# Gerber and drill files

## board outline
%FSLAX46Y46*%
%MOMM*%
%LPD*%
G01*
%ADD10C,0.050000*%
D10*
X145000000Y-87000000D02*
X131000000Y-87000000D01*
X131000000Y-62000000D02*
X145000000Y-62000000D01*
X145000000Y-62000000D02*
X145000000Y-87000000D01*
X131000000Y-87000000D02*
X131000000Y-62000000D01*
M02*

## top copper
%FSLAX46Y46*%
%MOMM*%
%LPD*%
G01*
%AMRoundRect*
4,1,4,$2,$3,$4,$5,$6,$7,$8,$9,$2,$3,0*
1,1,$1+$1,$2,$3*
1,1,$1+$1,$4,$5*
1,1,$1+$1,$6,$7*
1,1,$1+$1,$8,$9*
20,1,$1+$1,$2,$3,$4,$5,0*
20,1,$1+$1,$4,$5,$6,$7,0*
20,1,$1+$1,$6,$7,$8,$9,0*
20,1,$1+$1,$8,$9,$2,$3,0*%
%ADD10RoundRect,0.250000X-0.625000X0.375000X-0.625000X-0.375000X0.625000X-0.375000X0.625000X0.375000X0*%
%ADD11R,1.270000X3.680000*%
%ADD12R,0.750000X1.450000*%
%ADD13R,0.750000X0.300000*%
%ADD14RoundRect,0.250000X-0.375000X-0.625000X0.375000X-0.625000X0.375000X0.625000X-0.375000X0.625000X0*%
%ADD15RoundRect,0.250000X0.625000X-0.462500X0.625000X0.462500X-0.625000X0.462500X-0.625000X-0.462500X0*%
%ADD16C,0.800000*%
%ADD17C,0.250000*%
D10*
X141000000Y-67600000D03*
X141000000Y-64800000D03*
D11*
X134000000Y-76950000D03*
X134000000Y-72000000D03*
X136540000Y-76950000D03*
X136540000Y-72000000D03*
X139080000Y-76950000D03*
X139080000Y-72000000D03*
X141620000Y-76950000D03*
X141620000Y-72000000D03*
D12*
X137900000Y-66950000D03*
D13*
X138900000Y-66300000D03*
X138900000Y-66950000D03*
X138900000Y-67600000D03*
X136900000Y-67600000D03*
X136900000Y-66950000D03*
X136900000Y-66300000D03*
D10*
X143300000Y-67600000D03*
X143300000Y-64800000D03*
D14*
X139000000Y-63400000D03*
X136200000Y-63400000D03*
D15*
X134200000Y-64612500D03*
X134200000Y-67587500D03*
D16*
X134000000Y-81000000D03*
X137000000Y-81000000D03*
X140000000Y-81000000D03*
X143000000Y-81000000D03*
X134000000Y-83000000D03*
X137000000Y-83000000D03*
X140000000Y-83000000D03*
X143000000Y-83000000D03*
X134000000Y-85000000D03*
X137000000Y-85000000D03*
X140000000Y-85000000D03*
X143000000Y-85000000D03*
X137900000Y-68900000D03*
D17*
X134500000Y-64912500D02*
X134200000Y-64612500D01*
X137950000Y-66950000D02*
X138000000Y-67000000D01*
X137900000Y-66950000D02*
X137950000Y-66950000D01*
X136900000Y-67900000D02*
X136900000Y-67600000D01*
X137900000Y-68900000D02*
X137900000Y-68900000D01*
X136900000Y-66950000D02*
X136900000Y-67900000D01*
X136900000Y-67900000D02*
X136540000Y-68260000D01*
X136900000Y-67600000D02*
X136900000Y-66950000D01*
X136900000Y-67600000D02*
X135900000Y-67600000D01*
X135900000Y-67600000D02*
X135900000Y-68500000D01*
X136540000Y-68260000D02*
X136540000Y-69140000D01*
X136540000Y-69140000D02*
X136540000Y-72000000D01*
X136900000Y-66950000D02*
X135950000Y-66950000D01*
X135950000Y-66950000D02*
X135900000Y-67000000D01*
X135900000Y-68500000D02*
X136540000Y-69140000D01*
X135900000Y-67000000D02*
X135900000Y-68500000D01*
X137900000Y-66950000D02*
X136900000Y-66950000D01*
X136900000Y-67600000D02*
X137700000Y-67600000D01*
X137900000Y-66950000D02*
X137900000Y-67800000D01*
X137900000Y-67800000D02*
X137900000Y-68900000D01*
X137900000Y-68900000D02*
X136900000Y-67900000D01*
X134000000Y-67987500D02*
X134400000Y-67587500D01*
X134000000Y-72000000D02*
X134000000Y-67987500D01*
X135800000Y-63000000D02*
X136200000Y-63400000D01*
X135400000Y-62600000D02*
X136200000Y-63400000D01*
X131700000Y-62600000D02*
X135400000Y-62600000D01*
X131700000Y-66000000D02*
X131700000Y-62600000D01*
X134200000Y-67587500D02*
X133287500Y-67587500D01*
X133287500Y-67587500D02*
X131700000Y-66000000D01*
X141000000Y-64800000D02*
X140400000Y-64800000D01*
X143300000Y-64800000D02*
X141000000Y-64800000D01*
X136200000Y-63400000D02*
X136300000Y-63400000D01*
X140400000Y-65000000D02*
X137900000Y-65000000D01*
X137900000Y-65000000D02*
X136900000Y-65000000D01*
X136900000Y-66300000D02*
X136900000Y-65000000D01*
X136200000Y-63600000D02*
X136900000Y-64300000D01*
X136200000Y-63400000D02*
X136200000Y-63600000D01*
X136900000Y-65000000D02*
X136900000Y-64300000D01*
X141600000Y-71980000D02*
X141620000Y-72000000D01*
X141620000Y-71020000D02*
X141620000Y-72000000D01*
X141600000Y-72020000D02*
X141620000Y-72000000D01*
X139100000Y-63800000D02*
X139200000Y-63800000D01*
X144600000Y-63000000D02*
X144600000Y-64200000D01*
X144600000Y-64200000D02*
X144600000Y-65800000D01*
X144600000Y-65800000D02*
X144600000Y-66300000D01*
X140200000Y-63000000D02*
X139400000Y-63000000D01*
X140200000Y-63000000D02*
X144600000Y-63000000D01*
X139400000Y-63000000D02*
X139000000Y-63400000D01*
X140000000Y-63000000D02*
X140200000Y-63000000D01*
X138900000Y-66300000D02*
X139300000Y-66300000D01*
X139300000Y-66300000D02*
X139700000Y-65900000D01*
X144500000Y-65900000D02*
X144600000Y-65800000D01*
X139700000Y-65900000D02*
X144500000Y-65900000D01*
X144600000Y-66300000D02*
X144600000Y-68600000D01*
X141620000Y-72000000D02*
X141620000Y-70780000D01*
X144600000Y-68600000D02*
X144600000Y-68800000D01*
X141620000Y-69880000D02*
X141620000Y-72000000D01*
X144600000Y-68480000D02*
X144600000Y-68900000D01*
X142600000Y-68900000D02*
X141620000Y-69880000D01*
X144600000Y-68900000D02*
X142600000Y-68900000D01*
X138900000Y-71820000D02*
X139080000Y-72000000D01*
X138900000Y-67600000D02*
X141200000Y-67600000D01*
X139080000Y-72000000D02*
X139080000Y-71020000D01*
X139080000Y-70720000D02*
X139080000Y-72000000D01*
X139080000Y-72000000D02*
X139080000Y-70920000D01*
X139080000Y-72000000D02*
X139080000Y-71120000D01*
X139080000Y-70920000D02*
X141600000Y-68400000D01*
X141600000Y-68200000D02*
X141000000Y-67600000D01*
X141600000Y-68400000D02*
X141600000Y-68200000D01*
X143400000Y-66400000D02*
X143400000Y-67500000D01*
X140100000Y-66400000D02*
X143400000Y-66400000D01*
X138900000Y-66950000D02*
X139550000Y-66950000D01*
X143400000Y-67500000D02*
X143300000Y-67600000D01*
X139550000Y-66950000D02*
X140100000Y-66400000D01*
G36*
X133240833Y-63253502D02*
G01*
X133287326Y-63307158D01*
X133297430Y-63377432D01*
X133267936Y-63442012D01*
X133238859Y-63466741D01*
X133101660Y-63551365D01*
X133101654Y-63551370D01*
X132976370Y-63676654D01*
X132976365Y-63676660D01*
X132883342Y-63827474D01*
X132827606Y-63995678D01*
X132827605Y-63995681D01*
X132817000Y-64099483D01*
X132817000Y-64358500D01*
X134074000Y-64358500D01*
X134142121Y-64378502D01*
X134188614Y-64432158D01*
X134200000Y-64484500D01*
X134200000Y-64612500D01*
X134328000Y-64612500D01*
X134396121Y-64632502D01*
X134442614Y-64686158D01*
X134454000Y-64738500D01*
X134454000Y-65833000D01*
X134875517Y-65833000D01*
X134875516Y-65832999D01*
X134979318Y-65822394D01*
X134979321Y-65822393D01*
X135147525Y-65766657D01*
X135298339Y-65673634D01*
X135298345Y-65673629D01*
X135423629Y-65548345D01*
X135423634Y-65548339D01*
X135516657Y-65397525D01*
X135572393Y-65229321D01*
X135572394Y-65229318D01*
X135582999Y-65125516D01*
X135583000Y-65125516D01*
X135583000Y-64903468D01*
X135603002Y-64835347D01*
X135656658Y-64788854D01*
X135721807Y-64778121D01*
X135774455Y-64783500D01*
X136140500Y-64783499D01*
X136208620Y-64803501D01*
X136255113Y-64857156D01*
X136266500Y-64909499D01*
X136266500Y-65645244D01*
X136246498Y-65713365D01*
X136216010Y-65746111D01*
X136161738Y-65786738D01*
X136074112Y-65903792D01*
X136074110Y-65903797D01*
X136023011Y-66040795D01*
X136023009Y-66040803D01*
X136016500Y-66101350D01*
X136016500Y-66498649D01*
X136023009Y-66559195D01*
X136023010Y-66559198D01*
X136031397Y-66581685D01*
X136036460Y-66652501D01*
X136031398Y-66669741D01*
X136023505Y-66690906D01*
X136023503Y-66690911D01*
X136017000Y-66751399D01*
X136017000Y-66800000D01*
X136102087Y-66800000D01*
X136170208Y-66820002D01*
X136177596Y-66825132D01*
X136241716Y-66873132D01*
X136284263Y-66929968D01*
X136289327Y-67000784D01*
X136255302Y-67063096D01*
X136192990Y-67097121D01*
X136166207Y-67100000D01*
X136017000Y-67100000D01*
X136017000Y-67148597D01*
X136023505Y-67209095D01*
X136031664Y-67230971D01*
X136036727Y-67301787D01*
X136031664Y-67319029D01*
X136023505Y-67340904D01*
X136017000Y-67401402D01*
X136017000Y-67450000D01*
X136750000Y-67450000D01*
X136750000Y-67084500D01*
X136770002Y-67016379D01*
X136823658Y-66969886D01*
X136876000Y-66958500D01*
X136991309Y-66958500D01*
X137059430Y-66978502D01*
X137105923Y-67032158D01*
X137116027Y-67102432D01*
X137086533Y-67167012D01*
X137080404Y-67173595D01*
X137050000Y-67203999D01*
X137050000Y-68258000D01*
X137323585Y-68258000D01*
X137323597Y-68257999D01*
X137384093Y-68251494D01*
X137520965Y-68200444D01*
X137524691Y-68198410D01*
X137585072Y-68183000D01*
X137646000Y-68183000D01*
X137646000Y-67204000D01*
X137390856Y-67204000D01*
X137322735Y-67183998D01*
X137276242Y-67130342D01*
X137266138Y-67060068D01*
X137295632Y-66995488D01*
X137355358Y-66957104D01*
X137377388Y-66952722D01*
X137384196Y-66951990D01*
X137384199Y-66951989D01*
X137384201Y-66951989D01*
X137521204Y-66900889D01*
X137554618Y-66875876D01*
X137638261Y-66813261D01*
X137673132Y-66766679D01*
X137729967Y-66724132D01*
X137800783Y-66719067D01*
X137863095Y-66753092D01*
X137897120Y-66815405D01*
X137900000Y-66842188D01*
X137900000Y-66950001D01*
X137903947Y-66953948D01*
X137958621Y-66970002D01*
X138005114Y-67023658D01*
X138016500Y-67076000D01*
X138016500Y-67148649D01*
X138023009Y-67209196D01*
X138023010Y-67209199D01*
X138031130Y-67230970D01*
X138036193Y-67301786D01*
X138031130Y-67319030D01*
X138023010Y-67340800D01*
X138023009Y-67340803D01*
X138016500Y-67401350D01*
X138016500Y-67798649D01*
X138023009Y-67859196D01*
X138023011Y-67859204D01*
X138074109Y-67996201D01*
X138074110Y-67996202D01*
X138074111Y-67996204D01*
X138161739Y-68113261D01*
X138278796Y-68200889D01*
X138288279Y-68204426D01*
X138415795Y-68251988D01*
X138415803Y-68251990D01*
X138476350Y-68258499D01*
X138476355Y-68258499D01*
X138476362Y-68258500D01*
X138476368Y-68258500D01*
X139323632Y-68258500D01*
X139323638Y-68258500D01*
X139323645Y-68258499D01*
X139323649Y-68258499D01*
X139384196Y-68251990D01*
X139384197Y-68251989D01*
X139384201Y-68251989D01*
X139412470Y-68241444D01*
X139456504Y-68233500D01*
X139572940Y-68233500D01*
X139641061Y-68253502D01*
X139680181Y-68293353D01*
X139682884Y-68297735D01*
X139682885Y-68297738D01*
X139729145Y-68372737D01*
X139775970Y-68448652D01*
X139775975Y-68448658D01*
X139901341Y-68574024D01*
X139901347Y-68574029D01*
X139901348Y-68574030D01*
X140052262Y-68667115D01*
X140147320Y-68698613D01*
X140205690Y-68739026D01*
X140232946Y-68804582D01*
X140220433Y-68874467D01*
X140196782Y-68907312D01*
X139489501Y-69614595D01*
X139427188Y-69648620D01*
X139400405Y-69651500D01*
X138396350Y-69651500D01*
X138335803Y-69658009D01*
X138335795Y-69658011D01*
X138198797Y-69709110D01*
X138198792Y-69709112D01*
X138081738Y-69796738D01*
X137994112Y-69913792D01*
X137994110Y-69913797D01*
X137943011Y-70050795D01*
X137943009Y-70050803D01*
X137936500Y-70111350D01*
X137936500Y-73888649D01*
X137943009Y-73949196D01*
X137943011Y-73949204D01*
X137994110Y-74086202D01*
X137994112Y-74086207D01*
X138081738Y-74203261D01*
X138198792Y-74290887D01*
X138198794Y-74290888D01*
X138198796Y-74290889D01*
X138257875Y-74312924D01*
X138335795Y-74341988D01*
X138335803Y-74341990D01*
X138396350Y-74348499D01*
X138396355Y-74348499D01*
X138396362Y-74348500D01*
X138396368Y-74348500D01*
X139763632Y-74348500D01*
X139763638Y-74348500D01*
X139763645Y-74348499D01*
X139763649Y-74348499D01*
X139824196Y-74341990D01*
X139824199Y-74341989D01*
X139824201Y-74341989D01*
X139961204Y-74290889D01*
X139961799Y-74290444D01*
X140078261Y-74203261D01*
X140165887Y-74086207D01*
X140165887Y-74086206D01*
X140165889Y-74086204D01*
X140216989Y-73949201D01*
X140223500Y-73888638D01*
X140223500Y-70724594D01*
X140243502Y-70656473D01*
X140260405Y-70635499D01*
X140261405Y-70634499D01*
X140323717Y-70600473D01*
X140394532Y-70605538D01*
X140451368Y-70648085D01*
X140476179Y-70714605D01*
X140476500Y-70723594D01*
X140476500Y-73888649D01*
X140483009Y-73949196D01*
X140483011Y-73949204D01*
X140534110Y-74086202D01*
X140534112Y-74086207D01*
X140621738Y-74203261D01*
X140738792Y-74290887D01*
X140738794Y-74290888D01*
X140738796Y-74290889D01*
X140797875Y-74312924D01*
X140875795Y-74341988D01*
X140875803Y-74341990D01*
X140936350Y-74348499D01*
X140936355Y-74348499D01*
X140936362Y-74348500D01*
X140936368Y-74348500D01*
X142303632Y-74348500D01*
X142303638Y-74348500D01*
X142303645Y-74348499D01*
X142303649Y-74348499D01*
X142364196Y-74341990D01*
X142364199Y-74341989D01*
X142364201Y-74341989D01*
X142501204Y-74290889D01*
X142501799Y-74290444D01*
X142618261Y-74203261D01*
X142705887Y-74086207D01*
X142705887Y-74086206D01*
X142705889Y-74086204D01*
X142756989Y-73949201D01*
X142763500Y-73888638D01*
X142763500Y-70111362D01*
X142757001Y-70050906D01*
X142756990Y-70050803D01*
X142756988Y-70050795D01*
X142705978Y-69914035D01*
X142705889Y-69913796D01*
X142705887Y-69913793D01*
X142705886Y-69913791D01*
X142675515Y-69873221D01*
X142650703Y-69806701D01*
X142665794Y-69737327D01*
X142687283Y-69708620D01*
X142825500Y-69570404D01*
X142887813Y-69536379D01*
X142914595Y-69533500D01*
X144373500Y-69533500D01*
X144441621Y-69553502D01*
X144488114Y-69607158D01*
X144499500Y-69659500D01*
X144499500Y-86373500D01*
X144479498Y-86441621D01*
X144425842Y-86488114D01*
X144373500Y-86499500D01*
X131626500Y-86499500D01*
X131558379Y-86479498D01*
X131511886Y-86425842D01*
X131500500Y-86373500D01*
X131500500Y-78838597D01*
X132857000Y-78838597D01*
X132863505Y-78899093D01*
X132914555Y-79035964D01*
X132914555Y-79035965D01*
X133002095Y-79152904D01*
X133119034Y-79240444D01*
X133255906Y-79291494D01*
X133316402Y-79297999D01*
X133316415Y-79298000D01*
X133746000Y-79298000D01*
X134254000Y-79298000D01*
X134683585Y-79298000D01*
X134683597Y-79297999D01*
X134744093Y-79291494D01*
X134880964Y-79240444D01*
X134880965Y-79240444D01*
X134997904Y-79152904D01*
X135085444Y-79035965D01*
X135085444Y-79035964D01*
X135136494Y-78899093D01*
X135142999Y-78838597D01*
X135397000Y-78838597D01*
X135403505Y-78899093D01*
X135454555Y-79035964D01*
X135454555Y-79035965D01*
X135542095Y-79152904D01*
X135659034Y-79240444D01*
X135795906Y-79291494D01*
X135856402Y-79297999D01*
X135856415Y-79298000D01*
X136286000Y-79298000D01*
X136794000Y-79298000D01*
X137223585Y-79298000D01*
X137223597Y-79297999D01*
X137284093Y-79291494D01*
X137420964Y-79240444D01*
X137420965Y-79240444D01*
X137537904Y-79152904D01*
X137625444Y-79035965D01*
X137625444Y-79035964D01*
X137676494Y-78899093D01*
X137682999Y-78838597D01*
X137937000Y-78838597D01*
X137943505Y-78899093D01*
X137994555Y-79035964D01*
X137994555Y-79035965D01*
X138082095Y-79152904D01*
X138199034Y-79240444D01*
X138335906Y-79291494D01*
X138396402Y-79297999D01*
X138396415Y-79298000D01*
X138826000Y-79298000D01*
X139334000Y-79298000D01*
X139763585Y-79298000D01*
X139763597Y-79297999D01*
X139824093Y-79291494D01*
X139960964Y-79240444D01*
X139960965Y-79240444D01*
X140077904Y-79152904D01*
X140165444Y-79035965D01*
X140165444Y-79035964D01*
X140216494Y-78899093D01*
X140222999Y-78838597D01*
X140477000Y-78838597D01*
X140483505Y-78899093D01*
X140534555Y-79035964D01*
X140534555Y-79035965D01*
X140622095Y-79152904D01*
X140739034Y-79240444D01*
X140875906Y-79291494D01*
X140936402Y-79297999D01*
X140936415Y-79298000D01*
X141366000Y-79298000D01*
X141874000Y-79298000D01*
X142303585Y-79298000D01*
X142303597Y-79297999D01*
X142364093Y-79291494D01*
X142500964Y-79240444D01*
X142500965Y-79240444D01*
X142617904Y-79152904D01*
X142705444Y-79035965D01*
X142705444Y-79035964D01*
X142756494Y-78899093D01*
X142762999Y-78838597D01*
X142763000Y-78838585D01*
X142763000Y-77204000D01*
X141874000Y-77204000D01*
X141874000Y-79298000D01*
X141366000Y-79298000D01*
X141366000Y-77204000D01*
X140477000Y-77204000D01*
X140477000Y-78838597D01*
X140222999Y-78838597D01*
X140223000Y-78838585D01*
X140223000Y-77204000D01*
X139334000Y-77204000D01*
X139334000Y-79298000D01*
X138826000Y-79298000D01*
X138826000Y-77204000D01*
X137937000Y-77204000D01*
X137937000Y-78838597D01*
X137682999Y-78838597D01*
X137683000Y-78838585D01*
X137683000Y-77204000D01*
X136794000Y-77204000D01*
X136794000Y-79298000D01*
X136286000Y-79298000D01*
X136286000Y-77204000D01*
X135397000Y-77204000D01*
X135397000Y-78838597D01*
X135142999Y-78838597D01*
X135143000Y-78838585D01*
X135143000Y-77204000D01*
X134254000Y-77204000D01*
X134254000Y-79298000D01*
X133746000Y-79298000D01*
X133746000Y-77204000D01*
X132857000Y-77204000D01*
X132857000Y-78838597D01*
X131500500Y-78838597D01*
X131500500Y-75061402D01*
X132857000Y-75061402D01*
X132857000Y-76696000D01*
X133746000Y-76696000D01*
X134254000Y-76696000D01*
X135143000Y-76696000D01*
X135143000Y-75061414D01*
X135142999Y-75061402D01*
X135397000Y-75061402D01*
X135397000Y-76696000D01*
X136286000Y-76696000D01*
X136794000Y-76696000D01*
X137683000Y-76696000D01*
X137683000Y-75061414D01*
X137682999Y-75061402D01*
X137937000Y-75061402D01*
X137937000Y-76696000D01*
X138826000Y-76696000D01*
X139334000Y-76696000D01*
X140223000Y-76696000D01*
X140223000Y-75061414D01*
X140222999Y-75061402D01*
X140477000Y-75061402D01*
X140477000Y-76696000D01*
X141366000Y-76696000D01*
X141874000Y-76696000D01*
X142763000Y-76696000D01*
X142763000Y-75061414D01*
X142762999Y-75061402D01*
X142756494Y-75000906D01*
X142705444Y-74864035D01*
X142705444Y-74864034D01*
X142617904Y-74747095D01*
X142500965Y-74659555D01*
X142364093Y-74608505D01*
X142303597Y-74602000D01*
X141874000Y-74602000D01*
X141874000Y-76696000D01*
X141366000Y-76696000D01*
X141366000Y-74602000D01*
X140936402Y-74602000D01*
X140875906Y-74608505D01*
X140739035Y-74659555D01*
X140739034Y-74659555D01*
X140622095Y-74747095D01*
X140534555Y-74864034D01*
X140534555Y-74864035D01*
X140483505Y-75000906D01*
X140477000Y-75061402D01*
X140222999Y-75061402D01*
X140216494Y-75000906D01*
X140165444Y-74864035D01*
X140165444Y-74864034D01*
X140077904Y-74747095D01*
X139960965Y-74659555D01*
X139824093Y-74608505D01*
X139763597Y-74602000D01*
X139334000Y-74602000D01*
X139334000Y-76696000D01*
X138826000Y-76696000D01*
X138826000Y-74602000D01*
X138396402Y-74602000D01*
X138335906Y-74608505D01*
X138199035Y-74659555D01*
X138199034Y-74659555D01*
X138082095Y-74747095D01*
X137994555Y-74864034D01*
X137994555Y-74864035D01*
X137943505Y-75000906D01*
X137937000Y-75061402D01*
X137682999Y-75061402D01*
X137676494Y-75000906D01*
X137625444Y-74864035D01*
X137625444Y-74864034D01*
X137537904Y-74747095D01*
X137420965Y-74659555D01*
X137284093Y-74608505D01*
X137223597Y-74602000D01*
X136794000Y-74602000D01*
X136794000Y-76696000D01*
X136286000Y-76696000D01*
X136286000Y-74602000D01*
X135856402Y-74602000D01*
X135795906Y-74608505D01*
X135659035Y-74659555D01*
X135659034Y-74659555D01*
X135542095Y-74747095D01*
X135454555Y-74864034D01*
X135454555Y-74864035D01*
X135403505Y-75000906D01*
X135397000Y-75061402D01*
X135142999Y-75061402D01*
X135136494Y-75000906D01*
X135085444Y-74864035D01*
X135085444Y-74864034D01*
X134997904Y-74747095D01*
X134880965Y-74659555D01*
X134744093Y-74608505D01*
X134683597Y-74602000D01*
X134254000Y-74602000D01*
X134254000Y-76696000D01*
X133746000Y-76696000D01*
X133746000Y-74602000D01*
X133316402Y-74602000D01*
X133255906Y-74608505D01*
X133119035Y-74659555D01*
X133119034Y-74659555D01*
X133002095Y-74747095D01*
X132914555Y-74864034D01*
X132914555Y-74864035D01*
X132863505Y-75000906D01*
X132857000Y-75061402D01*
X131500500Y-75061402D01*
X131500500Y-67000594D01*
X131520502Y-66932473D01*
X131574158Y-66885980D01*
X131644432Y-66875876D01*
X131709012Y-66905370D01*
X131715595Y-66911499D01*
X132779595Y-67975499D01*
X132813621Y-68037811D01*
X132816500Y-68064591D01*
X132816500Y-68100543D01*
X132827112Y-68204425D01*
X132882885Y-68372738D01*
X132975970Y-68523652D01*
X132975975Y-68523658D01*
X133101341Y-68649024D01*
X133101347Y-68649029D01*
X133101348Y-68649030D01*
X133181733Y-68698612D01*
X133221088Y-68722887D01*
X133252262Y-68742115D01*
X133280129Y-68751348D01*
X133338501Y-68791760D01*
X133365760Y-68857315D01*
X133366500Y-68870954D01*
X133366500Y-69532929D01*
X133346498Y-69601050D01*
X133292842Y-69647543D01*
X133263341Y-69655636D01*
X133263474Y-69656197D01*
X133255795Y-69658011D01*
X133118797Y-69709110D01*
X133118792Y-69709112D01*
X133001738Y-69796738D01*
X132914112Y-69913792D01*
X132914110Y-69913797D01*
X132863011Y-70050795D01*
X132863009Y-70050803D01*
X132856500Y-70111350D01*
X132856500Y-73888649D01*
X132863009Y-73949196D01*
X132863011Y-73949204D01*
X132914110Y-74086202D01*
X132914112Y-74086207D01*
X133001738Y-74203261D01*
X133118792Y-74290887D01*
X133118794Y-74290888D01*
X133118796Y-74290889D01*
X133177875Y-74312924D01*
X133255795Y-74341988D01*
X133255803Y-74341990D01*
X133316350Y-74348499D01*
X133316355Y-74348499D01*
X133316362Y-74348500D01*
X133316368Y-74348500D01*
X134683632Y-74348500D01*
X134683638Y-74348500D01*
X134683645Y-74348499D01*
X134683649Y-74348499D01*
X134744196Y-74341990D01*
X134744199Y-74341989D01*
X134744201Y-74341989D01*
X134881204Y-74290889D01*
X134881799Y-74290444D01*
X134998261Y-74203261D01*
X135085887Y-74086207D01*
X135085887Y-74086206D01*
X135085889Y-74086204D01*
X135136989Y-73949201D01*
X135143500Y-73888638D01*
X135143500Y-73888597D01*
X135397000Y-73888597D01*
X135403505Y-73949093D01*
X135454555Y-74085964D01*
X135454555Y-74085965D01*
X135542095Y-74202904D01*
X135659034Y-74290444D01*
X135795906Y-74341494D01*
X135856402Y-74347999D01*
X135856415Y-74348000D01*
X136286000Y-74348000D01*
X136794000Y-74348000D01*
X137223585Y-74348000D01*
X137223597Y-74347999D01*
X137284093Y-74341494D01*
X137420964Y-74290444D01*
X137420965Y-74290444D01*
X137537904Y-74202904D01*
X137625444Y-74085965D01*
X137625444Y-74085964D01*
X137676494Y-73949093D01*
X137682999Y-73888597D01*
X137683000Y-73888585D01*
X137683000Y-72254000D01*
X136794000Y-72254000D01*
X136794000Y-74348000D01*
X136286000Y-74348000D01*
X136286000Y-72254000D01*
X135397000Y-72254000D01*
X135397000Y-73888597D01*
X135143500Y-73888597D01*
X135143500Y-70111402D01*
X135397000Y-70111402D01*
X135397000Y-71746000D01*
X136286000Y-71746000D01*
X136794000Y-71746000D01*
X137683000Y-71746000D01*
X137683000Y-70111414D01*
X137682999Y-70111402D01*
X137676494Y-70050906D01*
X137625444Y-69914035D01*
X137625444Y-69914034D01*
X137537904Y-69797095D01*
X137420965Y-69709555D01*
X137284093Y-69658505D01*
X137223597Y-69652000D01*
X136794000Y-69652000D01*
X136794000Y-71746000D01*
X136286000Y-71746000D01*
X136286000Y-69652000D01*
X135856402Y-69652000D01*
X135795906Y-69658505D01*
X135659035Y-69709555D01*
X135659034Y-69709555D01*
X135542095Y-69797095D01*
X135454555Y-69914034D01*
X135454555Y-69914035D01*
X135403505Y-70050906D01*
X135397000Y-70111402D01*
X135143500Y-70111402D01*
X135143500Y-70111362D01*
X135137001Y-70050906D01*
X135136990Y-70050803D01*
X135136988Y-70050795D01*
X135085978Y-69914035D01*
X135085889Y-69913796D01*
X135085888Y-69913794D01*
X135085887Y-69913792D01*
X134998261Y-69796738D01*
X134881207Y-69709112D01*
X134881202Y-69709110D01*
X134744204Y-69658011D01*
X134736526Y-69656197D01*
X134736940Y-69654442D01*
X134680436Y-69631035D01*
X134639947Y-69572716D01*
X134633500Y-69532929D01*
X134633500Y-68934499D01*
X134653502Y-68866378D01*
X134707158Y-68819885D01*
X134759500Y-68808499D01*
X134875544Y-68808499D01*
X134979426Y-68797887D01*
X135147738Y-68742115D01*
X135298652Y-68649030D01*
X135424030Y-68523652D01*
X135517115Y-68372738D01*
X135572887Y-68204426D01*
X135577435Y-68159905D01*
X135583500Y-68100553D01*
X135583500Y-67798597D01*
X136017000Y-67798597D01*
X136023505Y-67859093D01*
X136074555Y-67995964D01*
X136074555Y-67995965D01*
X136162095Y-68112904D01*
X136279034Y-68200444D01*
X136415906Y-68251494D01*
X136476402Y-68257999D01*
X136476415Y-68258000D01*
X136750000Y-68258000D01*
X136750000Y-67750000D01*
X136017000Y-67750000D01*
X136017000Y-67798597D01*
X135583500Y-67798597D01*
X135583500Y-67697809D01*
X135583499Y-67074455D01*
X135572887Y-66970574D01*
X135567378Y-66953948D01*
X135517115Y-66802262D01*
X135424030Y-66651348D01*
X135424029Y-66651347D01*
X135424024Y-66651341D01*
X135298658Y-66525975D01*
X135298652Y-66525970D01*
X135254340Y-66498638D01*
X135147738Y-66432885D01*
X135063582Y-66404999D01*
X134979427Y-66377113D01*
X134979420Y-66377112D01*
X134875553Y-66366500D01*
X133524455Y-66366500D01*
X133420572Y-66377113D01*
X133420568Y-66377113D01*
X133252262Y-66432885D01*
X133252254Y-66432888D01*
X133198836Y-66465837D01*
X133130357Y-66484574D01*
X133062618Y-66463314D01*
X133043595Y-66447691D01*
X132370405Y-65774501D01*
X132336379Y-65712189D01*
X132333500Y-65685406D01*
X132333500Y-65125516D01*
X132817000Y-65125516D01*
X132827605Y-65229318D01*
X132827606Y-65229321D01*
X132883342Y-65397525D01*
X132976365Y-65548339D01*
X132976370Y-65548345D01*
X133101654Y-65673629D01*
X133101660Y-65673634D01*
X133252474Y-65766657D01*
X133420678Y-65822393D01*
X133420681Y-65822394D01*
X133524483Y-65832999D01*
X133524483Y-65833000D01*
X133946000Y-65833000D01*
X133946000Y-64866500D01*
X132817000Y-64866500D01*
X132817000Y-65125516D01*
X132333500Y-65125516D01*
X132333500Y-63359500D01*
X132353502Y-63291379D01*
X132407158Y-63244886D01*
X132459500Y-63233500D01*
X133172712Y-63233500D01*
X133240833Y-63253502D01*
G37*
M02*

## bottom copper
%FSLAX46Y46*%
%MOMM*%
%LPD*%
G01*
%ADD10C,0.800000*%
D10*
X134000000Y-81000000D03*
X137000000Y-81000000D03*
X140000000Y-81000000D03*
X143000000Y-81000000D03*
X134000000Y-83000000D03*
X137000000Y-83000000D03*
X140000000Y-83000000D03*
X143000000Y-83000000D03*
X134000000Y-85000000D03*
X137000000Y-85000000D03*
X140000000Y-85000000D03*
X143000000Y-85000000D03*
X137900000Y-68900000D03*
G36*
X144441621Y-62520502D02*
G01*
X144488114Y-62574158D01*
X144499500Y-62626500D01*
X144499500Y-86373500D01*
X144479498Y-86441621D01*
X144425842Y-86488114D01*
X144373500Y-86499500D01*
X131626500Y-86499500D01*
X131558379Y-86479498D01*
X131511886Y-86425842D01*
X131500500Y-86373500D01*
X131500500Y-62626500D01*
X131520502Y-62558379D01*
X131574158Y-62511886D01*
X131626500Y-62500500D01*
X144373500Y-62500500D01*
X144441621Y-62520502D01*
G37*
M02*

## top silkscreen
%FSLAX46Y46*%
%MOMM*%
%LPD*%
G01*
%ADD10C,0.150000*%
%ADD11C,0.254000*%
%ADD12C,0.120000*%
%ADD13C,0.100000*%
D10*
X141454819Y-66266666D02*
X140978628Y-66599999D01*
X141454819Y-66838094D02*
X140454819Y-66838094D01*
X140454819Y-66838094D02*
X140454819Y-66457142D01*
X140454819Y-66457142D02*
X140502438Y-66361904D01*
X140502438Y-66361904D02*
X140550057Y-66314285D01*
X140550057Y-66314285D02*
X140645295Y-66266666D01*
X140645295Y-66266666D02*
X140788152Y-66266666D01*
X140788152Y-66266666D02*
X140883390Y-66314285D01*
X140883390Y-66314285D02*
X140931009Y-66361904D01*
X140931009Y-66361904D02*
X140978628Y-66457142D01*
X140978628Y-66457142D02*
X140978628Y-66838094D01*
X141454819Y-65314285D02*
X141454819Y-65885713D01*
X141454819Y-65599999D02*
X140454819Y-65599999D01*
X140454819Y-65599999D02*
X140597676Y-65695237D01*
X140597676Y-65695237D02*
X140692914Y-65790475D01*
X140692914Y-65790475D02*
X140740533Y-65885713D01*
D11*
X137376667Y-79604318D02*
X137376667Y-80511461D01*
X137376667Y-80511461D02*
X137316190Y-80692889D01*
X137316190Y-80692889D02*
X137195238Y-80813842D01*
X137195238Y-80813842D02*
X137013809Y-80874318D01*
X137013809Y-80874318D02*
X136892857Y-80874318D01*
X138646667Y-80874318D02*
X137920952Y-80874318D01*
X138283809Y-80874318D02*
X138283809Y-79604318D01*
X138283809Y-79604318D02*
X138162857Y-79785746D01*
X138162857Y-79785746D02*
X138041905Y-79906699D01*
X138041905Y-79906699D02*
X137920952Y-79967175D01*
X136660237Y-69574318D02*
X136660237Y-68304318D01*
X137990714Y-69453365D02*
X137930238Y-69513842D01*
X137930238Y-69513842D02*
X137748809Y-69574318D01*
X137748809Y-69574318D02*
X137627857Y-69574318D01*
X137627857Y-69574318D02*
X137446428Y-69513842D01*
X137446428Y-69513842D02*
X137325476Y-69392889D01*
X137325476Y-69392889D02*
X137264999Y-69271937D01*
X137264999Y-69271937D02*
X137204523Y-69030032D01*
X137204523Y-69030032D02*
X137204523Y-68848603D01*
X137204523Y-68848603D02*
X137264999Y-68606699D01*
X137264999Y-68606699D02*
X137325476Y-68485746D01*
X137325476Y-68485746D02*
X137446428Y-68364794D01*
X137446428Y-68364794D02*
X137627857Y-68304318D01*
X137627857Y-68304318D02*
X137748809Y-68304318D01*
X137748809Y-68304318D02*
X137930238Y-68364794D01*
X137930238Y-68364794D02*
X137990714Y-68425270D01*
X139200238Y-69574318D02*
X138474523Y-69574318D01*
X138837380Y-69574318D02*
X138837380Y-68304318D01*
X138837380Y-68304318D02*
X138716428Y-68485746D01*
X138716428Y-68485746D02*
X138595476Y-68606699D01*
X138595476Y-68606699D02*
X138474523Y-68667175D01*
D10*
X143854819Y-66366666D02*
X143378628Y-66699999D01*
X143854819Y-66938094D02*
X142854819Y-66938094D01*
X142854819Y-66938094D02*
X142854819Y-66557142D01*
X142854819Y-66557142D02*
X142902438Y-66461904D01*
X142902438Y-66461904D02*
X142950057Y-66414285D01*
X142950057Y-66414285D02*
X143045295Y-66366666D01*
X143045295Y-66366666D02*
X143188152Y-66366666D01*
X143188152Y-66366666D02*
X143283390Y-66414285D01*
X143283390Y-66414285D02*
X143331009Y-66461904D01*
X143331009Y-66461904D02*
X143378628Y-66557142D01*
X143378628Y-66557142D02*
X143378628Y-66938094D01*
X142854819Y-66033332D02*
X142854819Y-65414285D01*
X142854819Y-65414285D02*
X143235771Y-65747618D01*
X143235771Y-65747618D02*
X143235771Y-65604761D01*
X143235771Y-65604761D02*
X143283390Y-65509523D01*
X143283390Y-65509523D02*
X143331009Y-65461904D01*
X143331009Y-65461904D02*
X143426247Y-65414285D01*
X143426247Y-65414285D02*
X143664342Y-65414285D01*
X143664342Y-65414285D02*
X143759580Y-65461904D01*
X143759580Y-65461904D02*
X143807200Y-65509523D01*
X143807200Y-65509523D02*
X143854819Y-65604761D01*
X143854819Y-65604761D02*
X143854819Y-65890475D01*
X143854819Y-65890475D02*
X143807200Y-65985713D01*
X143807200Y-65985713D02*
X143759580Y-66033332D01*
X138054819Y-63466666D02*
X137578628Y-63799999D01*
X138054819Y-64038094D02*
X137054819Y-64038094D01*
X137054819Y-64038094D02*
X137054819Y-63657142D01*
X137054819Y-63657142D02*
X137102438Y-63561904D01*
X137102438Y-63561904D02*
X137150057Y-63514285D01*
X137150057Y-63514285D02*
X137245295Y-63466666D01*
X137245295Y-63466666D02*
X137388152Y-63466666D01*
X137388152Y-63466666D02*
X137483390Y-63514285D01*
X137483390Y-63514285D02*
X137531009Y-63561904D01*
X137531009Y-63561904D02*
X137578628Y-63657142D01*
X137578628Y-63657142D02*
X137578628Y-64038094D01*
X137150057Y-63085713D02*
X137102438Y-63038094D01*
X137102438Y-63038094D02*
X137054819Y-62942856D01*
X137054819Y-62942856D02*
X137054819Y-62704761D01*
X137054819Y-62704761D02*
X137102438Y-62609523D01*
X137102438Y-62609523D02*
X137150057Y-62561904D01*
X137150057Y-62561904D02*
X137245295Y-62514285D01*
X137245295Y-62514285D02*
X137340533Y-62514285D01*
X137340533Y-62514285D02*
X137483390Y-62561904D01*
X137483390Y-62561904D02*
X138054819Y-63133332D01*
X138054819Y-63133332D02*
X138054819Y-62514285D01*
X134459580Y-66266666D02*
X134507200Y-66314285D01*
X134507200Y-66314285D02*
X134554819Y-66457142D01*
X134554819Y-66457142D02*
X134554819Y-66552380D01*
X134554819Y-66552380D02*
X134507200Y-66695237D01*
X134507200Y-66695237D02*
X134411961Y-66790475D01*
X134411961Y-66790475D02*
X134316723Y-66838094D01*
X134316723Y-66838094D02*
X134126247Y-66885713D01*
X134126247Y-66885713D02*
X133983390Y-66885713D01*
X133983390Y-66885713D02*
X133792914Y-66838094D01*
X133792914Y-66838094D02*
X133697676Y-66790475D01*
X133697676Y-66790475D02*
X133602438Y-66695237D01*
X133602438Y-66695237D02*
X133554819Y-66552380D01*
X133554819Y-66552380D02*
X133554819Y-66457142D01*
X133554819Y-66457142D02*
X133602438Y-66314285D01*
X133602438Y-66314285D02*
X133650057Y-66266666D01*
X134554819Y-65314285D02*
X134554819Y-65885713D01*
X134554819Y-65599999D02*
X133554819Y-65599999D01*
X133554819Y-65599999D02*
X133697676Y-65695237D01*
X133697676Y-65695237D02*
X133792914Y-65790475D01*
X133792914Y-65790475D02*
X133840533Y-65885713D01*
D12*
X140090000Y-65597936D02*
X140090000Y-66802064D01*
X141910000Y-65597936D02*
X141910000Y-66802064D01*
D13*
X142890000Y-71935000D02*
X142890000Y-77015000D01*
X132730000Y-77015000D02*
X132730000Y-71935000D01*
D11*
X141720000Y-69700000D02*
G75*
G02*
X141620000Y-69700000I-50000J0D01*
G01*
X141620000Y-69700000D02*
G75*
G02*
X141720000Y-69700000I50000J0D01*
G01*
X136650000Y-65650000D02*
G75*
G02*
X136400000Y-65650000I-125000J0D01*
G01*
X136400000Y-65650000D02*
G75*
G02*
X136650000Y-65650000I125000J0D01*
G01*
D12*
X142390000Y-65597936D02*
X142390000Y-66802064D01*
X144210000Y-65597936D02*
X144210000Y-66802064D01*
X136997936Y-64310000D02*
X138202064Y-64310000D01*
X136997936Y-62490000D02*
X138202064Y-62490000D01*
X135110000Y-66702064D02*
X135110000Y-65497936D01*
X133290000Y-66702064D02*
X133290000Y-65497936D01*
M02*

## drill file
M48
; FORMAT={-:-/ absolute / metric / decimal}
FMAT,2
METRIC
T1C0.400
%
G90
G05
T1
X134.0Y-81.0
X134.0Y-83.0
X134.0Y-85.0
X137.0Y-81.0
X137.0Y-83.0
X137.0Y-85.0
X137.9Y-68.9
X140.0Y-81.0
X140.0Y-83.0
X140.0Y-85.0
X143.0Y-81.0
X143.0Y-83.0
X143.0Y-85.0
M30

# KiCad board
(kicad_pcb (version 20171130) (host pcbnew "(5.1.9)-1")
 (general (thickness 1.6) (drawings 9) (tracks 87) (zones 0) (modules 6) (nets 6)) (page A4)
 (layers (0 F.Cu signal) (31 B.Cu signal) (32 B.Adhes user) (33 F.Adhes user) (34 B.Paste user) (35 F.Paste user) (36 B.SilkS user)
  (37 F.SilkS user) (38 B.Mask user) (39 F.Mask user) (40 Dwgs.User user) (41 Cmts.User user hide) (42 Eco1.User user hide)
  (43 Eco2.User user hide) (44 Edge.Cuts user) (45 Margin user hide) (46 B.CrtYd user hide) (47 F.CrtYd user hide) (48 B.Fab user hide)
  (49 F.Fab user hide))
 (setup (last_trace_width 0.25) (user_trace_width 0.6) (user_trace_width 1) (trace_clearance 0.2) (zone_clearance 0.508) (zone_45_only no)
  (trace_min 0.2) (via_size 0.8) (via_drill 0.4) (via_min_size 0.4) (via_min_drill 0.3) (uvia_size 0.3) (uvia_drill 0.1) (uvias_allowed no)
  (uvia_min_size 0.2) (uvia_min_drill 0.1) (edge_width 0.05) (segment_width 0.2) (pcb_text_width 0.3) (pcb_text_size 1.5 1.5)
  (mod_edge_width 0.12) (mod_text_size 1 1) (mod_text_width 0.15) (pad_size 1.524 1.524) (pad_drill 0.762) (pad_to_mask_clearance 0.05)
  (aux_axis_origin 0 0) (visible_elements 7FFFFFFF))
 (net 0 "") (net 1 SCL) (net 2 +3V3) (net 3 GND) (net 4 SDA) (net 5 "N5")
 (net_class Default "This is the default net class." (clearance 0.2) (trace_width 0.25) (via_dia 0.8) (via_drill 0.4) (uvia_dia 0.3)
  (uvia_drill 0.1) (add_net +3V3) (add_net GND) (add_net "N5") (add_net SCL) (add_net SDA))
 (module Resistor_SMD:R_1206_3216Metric (layer F.Cu) (at 141 66.2 270)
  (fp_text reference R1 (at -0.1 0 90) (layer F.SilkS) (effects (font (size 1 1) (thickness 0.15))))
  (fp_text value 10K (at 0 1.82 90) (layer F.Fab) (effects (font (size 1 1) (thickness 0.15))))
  (fp_line (start -0.602064 0.91) (end 0.602064 0.91) (layer F.SilkS) (width 0.12))
  (fp_line (start -0.602064 -0.91) (end 0.602064 -0.91) (layer F.SilkS) (width 0.12))
  (pad 2 smd roundrect (at 1.4 0 270) (size 1.25 1.75) (layers F.Cu F.Paste F.Mask) (roundrect_rratio 0.2) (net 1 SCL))
  (pad 1 smd roundrect (at -1.4 0 270) (size 1.25 1.75) (layers F.Cu F.Paste F.Mask) (roundrect_rratio 0.2) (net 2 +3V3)))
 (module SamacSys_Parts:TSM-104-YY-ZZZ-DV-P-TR (layer F.Cu) (at 137.81 74.475)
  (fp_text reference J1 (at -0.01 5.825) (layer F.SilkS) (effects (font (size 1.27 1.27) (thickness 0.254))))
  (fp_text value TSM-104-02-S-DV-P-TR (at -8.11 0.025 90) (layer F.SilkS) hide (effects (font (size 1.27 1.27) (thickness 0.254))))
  (fp_line (start 5.08 -2.54) (end 5.08 2.54) (layer F.SilkS) (width 0.1))
  (fp_line (start -5.08 2.54) (end -5.08 -2.54) (layer F.SilkS) (width 0.1))
  (fp_circle (center 3.86 -4.775) (end 3.81 -4.775) (layer F.SilkS) (width 0.254))
  (pad 8 smd rect (at -3.81 2.475) (size 1.27 3.68) (layers F.Cu F.Paste F.Mask) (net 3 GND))
  (pad 7 smd rect (at -3.81 -2.475) (size 1.27 3.68) (layers F.Cu F.Paste F.Mask) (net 2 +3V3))
  (pad 6 smd rect (at -1.27 2.475) (size 1.27 3.68) (layers F.Cu F.Paste F.Mask) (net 3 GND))
  (pad 5 smd rect (at -1.27 -2.475) (size 1.27 3.68) (layers F.Cu F.Paste F.Mask) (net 3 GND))
  (pad 4 smd rect (at 1.27 2.475) (size 1.27 3.68) (layers F.Cu F.Paste F.Mask) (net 3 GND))
  (pad 3 smd rect (at 1.27 -2.475) (size 1.27 3.68) (layers F.Cu F.Paste F.Mask) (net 1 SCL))
  (pad 2 smd rect (at 3.81 2.475) (size 1.27 3.68) (layers F.Cu F.Paste F.Mask) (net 3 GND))
  (pad 1 smd rect (at 3.81 -2.475) (size 1.27 3.68) (layers F.Cu F.Paste F.Mask) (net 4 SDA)))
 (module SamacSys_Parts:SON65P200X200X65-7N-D (layer F.Cu) (at 137.9 66.95)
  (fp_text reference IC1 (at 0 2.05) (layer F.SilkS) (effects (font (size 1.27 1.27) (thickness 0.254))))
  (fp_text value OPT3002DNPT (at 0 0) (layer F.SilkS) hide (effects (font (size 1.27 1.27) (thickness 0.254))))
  (fp_circle (center -1.375 -1.3) (end -1.25 -1.3) (layer F.SilkS) (width 0.254))
  (pad 7 smd rect (at 0 0) (size 0.75 1.45) (layers F.Cu F.Paste F.Mask) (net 3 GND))
  (pad 6 smd rect (at 1 -0.65 90) (size 0.3 0.75) (layers F.Cu F.Paste F.Mask) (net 4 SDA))
  (pad 5 smd rect (at 1 0 90) (size 0.3 0.75) (layers F.Cu F.Paste F.Mask) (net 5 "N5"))
  (pad 4 smd rect (at 1 0.65 90) (size 0.3 0.75) (layers F.Cu F.Paste F.Mask) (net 1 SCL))
  (pad 3 smd rect (at -1 0.65 90) (size 0.3 0.75) (layers F.Cu F.Paste F.Mask) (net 3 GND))
  (pad 2 smd rect (at -1 0 90) (size 0.3 0.75) (layers F.Cu F.Paste F.Mask) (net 3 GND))
  (pad 1 smd rect (at -1 -0.65 90) (size 0.3 0.75) (layers F.Cu F.Paste F.Mask) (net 2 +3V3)))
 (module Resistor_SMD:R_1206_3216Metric (layer F.Cu) (at 143.3 66.2 270)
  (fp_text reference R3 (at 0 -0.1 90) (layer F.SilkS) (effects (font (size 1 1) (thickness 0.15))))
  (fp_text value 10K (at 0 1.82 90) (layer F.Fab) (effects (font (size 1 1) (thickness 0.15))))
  (fp_line (start -0.602064 0.91) (end 0.602064 0.91) (layer F.SilkS) (width 0.12))
  (fp_line (start -0.602064 -0.91) (end 0.602064 -0.91) (layer F.SilkS) (width 0.12))
  (pad 2 smd roundrect (at 1.4 0 270) (size 1.25 1.75) (layers F.Cu F.Paste F.Mask) (roundrect_rratio 0.2) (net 5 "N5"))
  (pad 1 smd roundrect (at -1.4 0 270) (size 1.25 1.75) (layers F.Cu F.Paste F.Mask) (roundrect_rratio 0.2) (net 2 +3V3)))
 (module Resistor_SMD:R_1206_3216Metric (layer F.Cu) (at 137.6 63.4)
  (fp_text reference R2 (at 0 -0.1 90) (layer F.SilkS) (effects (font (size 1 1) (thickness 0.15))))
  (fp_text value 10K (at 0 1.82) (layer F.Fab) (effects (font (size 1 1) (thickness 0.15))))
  (fp_line (start -0.602064 0.91) (end 0.602064 0.91) (layer F.SilkS) (width 0.12))
  (fp_line (start -0.602064 -0.91) (end 0.602064 -0.91) (layer F.SilkS) (width 0.12))
  (pad 2 smd roundrect (at 1.4 0) (size 1.25 1.75) (layers F.Cu F.Paste F.Mask) (roundrect_rratio 0.2) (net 4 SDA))
  (pad 1 smd roundrect (at -1.4 0) (size 1.25 1.75) (layers F.Cu F.Paste F.Mask) (roundrect_rratio 0.2) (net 2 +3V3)))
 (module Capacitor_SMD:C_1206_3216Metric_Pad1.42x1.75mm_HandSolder (layer F.Cu) (at 134.2 66.1 90)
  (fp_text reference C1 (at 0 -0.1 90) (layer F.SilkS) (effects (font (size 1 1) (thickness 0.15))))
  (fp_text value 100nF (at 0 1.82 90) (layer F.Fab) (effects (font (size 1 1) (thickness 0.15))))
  (fp_line (start -0.602064 0.91) (end 0.602064 0.91) (layer F.SilkS) (width 0.12))
  (fp_line (start -0.602064 -0.91) (end 0.602064 -0.91) (layer F.SilkS) (width 0.12))
  (pad 2 smd roundrect (at 1.4875 0 90) (size 1.425 1.75) (layers F.Cu F.Paste F.Mask) (roundrect_rratio 0.1754385964912281) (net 3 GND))
  (pad 1 smd roundrect (at -1.4875 0 90) (size 1.425 1.75) (layers F.Cu F.Paste F.Mask) (roundrect_rratio 0.1754385964912281) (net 2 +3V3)))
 (gr_line (start 145 87) (end 131 87) (layer Edge.Cuts) (width 0.05))
 (gr_line (start 131 62) (end 145 62) (layer Edge.Cuts) (width 0.05))
 (gr_line (start 145 62) (end 145 87) (layer Edge.Cuts) (width 0.05))
 (gr_line (start 131 87) (end 131 62) (layer Edge.Cuts) (width 0.05))
 (segment (start 134.5 64.9125) (end 134.2 64.6125) (width 0.25) (layer F.Cu) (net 3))
 (segment (start 137.95 66.95) (end 138 67) (width 0.25) (layer F.Cu) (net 3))
 (segment (start 137.9 66.95) (end 137.95 66.95) (width 0.25) (layer F.Cu) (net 3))
 (segment (start 136.9 67.9) (end 136.9 67.6) (width 0.25) (layer F.Cu) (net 3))
 (segment (start 137.9 68.9) (end 137.9 68.9) (width 0.25) (layer F.Cu) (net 3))
 (segment (start 136.9 66.95) (end 136.9 67.9) (width 0.25) (layer F.Cu) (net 3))
 (segment (start 136.9 67.9) (end 136.54 68.26) (width 0.25) (layer F.Cu) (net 3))
 (segment (start 136.9 67.6) (end 136.9 66.95) (width 0.25) (layer F.Cu) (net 3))
 (segment (start 136.9 67.6) (end 135.9 67.6) (width 0.25) (layer F.Cu) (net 3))
 (segment (start 135.9 67.6) (end 135.9 68.5) (width 0.25) (layer F.Cu) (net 3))
 (segment (start 136.54 68.26) (end 136.54 69.14) (width 0.25) (layer F.Cu) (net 3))
 (segment (start 136.54 69.14) (end 136.54 72) (width 0.25) (layer F.Cu) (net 3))
 (segment (start 136.9 66.95) (end 135.95 66.95) (width 0.25) (layer F.Cu) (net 3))
 (segment (start 135.95 66.95) (end 135.9 67) (width 0.25) (layer F.Cu) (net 3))
 (segment (start 135.9 68.5) (end 136.54 69.14) (width 0.25) (layer F.Cu) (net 3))
 (segment (start 135.9 67) (end 135.9 68.5) (width 0.25) (layer F.Cu) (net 3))
 (segment (start 137.9 66.95) (end 136.9 66.95) (width 0.25) (layer F.Cu) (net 3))
 (segment (start 136.9 67.6) (end 137.7 67.6) (width 0.25) (layer F.Cu) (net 3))
 (segment (start 137.9 66.95) (end 137.9 67.8) (width 0.25) (layer F.Cu) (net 3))
 (segment (start 137.9 67.8) (end 137.9 68.9) (width 0.25) (layer F.Cu) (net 3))
 (via (at 134 81) (size 0.8) (drill 0.4) (layers F.Cu B.Cu) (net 3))
 (via (at 137 81) (size 0.8) (drill 0.4) (layers F.Cu B.Cu) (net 3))
 (via (at 140 81) (size 0.8) (drill 0.4) (layers F.Cu B.Cu) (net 3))
 (via (at 143 81) (size 0.8) (drill 0.4) (layers F.Cu B.Cu) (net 3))
 (via (at 134 83) (size 0.8) (drill 0.4) (layers F.Cu B.Cu) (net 3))
 (via (at 137 83) (size 0.8) (drill 0.4) (layers F.Cu B.Cu) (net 3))
 (via (at 140 83) (size 0.8) (drill 0.4) (layers F.Cu B.Cu) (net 3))
 (via (at 143 83) (size 0.8) (drill 0.4) (layers F.Cu B.Cu) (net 3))
 (via (at 134 85) (size 0.8) (drill 0.4) (layers F.Cu B.Cu) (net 3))
 (via (at 137 85) (size 0.8) (drill 0.4) (layers F.Cu B.Cu) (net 3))
 (via (at 140 85) (size 0.8) (drill 0.4) (layers F.Cu B.Cu) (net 3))
 (via (at 143 85) (size 0.8) (drill 0.4) (layers F.Cu B.Cu) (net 3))
 (segment (start 137.9 68.9) (end 136.9 67.9) (width 0.25) (layer F.Cu) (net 3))
 (via (at 137.9 68.9) (size 0.8) (drill 0.4) (layers F.Cu B.Cu) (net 3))
 (segment (start 134 67.9875) (end 134.4 67.5875) (width 0.25) (layer F.Cu) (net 2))
 (segment (start 134 72) (end 134 67.9875) (width 0.25) (layer F.Cu) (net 2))
 (segment (start 135.8 63) (end 136.2 63.4) (width 0.25) (layer F.Cu) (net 2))
 (segment (start 135.4 62.6) (end 136.2 63.4) (width 0.25) (layer F.Cu) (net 2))
 (segment (start 131.7 62.6) (end 135.4 62.6) (width 0.25) (layer F.Cu) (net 2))
 (segment (start 131.7 66) (end 131.7 62.6) (width 0.25) (layer F.Cu) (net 2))
 (segment (start 134.2 67.5875) (end 133.2875 67.5875) (width 0.25) (layer F.Cu) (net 2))
 (segment (start 133.2875 67.5875) (end 131.7 66) (width 0.25) (layer F.Cu) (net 2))
 (segment (start 141 64.8) (end 140.4 64.8) (width 0.25) (layer F.Cu) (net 2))
 (segment (start 143.3 64.8) (end 141 64.8) (width 0.25) (layer F.Cu) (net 2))
 (segment (start 136.2 63.4) (end 136.3 63.4) (width 0.25) (layer F.Cu) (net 2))
 (segment (start 140.4 65) (end 137.9 65) (width 0.25) (layer F.Cu) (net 2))
 (segment (start 137.9 65) (end 136.9 65) (width 0.25) (layer F.Cu) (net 2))
 (segment (start 136.9 66.3) (end 136.9 65) (width 0.25) (layer F.Cu) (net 2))
 (segment (start 136.2 63.6) (end 136.9 64.3) (width 0.25) (layer F.Cu) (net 2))
 (segment (start 136.2 63.4) (end 136.2 63.6) (width 0.25) (layer F.Cu) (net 2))
 (segment (start 136.9 65) (end 136.9 64.3) (width 0.25) (layer F.Cu) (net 2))
 (segment (start 141.6 71.98) (end 141.62 72) (width 0.25) (layer F.Cu) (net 4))
 (segment (start 141.62 71.02) (end 141.62 72) (width 0.25) (layer F.Cu) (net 4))
 (segment (start 141.6 72.02) (end 141.62 72) (width 0.25) (layer F.Cu) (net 4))
 (segment (start 139.1 63.8) (end 139.2 63.8) (width 0.25) (layer F.Cu) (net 4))
 (segment (start 144.6 63) (end 144.6 64.2) (width 0.25) (layer F.Cu) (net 4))
 (segment (start 144.6 64.2) (end 144.6 65.8) (width 0.25) (layer F.Cu) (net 4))
 (segment (start 144.6 65.8) (end 144.6 66.3) (width 0.25) (layer F.Cu) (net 4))
 (segment (start 140.2 63) (end 139.4 63) (width 0.25) (layer F.Cu) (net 4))
 (segment (start 140.2 63) (end 144.6 63) (width 0.25) (layer F.Cu) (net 4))
 (segment (start 139.4 63) (end 139 63.4) (width 0.25) (layer F.Cu) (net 4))
 (segment (start 140 63) (end 140.2 63) (width 0.25) (layer F.Cu) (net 4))
 (segment (start 138.9 66.3) (end 139.3 66.3) (width 0.25) (layer F.Cu) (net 4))
 (segment (start 139.3 66.3) (end 139.7 65.9) (width 0.25) (layer F.Cu) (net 4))
 (segment (start 144.5 65.9) (end 144.6 65.8) (width 0.25) (layer F.Cu) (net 4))
 (segment (start 139.7 65.9) (end 144.5 65.9) (width 0.25) (layer F.Cu) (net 4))
 (segment (start 144.6 66.3) (end 144.6 68.6) (width 0.25) (layer F.Cu) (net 4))
 (segment (start 141.62 72) (end 141.62 70.78) (width 0.25) (layer F.Cu) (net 4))
 (segment (start 144.6 68.6) (end 144.6 68.8) (width 0.25) (layer F.Cu) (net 4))
 (segment (start 141.62 69.88) (end 141.62 72) (width 0.25) (layer F.Cu) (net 4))
 (segment (start 144.6 68.48) (end 144.6 68.9) (width 0.25) (layer F.Cu) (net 4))
 (segment (start 142.6 68.9) (end 141.62 69.88) (width 0.25) (layer F.Cu) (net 4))
 (segment (start 144.6 68.9) (end 142.6 68.9) (width 0.25) (layer F.Cu) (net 4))
 (segment (start 138.9 71.82) (end 139.08 72) (width 0.25) (layer F.Cu) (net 1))
 (segment (start 138.9 67.6) (end 141.2 67.6) (width 0.25) (layer F.Cu) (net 1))
 (segment (start 139.08 72) (end 139.08 71.02) (width 0.25) (layer F.Cu) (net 1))
 (segment (start 139.08 70.72) (end 139.08 72) (width 0.25) (layer F.Cu) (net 1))
 (segment (start 139.08 72) (end 139.08 70.92) (width 0.25) (layer F.Cu) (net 1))
 (segment (start 139.08 72) (end 139.08 71.12) (width 0.25) (layer F.Cu) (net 1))
 (segment (start 139.08 70.92) (end 141.6 68.4) (width 0.25) (layer F.Cu) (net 1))
 (segment (start 141.6 68.2) (end 141 67.6) (width 0.25) (layer F.Cu) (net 1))
 (segment (start 141.6 68.4) (end 141.6 68.2) (width 0.25) (layer F.Cu) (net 1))
 (segment (start 143.4 66.4) (end 143.4 67.5) (width 0.25) (layer F.Cu) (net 5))
 (segment (start 140.1 66.4) (end 143.4 66.4) (width 0.25) (layer F.Cu) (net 5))
 (segment (start 138.9 66.95) (end 139.55 66.95) (width 0.25) (layer F.Cu) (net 5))
 (segment (start 143.4 67.5) (end 143.3 67.6) (width 0.25) (layer F.Cu) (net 5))
 (segment (start 139.55 66.95) (end 140.1 66.4) (width 0.25) (layer F.Cu) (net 5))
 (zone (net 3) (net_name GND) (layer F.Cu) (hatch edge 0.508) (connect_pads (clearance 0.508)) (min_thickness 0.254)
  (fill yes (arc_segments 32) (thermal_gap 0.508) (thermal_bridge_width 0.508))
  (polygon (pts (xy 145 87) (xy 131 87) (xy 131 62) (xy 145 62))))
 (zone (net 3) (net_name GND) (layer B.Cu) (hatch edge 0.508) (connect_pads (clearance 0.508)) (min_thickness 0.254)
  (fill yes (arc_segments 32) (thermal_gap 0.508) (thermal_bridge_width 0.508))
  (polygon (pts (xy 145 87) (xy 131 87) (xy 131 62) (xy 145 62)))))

